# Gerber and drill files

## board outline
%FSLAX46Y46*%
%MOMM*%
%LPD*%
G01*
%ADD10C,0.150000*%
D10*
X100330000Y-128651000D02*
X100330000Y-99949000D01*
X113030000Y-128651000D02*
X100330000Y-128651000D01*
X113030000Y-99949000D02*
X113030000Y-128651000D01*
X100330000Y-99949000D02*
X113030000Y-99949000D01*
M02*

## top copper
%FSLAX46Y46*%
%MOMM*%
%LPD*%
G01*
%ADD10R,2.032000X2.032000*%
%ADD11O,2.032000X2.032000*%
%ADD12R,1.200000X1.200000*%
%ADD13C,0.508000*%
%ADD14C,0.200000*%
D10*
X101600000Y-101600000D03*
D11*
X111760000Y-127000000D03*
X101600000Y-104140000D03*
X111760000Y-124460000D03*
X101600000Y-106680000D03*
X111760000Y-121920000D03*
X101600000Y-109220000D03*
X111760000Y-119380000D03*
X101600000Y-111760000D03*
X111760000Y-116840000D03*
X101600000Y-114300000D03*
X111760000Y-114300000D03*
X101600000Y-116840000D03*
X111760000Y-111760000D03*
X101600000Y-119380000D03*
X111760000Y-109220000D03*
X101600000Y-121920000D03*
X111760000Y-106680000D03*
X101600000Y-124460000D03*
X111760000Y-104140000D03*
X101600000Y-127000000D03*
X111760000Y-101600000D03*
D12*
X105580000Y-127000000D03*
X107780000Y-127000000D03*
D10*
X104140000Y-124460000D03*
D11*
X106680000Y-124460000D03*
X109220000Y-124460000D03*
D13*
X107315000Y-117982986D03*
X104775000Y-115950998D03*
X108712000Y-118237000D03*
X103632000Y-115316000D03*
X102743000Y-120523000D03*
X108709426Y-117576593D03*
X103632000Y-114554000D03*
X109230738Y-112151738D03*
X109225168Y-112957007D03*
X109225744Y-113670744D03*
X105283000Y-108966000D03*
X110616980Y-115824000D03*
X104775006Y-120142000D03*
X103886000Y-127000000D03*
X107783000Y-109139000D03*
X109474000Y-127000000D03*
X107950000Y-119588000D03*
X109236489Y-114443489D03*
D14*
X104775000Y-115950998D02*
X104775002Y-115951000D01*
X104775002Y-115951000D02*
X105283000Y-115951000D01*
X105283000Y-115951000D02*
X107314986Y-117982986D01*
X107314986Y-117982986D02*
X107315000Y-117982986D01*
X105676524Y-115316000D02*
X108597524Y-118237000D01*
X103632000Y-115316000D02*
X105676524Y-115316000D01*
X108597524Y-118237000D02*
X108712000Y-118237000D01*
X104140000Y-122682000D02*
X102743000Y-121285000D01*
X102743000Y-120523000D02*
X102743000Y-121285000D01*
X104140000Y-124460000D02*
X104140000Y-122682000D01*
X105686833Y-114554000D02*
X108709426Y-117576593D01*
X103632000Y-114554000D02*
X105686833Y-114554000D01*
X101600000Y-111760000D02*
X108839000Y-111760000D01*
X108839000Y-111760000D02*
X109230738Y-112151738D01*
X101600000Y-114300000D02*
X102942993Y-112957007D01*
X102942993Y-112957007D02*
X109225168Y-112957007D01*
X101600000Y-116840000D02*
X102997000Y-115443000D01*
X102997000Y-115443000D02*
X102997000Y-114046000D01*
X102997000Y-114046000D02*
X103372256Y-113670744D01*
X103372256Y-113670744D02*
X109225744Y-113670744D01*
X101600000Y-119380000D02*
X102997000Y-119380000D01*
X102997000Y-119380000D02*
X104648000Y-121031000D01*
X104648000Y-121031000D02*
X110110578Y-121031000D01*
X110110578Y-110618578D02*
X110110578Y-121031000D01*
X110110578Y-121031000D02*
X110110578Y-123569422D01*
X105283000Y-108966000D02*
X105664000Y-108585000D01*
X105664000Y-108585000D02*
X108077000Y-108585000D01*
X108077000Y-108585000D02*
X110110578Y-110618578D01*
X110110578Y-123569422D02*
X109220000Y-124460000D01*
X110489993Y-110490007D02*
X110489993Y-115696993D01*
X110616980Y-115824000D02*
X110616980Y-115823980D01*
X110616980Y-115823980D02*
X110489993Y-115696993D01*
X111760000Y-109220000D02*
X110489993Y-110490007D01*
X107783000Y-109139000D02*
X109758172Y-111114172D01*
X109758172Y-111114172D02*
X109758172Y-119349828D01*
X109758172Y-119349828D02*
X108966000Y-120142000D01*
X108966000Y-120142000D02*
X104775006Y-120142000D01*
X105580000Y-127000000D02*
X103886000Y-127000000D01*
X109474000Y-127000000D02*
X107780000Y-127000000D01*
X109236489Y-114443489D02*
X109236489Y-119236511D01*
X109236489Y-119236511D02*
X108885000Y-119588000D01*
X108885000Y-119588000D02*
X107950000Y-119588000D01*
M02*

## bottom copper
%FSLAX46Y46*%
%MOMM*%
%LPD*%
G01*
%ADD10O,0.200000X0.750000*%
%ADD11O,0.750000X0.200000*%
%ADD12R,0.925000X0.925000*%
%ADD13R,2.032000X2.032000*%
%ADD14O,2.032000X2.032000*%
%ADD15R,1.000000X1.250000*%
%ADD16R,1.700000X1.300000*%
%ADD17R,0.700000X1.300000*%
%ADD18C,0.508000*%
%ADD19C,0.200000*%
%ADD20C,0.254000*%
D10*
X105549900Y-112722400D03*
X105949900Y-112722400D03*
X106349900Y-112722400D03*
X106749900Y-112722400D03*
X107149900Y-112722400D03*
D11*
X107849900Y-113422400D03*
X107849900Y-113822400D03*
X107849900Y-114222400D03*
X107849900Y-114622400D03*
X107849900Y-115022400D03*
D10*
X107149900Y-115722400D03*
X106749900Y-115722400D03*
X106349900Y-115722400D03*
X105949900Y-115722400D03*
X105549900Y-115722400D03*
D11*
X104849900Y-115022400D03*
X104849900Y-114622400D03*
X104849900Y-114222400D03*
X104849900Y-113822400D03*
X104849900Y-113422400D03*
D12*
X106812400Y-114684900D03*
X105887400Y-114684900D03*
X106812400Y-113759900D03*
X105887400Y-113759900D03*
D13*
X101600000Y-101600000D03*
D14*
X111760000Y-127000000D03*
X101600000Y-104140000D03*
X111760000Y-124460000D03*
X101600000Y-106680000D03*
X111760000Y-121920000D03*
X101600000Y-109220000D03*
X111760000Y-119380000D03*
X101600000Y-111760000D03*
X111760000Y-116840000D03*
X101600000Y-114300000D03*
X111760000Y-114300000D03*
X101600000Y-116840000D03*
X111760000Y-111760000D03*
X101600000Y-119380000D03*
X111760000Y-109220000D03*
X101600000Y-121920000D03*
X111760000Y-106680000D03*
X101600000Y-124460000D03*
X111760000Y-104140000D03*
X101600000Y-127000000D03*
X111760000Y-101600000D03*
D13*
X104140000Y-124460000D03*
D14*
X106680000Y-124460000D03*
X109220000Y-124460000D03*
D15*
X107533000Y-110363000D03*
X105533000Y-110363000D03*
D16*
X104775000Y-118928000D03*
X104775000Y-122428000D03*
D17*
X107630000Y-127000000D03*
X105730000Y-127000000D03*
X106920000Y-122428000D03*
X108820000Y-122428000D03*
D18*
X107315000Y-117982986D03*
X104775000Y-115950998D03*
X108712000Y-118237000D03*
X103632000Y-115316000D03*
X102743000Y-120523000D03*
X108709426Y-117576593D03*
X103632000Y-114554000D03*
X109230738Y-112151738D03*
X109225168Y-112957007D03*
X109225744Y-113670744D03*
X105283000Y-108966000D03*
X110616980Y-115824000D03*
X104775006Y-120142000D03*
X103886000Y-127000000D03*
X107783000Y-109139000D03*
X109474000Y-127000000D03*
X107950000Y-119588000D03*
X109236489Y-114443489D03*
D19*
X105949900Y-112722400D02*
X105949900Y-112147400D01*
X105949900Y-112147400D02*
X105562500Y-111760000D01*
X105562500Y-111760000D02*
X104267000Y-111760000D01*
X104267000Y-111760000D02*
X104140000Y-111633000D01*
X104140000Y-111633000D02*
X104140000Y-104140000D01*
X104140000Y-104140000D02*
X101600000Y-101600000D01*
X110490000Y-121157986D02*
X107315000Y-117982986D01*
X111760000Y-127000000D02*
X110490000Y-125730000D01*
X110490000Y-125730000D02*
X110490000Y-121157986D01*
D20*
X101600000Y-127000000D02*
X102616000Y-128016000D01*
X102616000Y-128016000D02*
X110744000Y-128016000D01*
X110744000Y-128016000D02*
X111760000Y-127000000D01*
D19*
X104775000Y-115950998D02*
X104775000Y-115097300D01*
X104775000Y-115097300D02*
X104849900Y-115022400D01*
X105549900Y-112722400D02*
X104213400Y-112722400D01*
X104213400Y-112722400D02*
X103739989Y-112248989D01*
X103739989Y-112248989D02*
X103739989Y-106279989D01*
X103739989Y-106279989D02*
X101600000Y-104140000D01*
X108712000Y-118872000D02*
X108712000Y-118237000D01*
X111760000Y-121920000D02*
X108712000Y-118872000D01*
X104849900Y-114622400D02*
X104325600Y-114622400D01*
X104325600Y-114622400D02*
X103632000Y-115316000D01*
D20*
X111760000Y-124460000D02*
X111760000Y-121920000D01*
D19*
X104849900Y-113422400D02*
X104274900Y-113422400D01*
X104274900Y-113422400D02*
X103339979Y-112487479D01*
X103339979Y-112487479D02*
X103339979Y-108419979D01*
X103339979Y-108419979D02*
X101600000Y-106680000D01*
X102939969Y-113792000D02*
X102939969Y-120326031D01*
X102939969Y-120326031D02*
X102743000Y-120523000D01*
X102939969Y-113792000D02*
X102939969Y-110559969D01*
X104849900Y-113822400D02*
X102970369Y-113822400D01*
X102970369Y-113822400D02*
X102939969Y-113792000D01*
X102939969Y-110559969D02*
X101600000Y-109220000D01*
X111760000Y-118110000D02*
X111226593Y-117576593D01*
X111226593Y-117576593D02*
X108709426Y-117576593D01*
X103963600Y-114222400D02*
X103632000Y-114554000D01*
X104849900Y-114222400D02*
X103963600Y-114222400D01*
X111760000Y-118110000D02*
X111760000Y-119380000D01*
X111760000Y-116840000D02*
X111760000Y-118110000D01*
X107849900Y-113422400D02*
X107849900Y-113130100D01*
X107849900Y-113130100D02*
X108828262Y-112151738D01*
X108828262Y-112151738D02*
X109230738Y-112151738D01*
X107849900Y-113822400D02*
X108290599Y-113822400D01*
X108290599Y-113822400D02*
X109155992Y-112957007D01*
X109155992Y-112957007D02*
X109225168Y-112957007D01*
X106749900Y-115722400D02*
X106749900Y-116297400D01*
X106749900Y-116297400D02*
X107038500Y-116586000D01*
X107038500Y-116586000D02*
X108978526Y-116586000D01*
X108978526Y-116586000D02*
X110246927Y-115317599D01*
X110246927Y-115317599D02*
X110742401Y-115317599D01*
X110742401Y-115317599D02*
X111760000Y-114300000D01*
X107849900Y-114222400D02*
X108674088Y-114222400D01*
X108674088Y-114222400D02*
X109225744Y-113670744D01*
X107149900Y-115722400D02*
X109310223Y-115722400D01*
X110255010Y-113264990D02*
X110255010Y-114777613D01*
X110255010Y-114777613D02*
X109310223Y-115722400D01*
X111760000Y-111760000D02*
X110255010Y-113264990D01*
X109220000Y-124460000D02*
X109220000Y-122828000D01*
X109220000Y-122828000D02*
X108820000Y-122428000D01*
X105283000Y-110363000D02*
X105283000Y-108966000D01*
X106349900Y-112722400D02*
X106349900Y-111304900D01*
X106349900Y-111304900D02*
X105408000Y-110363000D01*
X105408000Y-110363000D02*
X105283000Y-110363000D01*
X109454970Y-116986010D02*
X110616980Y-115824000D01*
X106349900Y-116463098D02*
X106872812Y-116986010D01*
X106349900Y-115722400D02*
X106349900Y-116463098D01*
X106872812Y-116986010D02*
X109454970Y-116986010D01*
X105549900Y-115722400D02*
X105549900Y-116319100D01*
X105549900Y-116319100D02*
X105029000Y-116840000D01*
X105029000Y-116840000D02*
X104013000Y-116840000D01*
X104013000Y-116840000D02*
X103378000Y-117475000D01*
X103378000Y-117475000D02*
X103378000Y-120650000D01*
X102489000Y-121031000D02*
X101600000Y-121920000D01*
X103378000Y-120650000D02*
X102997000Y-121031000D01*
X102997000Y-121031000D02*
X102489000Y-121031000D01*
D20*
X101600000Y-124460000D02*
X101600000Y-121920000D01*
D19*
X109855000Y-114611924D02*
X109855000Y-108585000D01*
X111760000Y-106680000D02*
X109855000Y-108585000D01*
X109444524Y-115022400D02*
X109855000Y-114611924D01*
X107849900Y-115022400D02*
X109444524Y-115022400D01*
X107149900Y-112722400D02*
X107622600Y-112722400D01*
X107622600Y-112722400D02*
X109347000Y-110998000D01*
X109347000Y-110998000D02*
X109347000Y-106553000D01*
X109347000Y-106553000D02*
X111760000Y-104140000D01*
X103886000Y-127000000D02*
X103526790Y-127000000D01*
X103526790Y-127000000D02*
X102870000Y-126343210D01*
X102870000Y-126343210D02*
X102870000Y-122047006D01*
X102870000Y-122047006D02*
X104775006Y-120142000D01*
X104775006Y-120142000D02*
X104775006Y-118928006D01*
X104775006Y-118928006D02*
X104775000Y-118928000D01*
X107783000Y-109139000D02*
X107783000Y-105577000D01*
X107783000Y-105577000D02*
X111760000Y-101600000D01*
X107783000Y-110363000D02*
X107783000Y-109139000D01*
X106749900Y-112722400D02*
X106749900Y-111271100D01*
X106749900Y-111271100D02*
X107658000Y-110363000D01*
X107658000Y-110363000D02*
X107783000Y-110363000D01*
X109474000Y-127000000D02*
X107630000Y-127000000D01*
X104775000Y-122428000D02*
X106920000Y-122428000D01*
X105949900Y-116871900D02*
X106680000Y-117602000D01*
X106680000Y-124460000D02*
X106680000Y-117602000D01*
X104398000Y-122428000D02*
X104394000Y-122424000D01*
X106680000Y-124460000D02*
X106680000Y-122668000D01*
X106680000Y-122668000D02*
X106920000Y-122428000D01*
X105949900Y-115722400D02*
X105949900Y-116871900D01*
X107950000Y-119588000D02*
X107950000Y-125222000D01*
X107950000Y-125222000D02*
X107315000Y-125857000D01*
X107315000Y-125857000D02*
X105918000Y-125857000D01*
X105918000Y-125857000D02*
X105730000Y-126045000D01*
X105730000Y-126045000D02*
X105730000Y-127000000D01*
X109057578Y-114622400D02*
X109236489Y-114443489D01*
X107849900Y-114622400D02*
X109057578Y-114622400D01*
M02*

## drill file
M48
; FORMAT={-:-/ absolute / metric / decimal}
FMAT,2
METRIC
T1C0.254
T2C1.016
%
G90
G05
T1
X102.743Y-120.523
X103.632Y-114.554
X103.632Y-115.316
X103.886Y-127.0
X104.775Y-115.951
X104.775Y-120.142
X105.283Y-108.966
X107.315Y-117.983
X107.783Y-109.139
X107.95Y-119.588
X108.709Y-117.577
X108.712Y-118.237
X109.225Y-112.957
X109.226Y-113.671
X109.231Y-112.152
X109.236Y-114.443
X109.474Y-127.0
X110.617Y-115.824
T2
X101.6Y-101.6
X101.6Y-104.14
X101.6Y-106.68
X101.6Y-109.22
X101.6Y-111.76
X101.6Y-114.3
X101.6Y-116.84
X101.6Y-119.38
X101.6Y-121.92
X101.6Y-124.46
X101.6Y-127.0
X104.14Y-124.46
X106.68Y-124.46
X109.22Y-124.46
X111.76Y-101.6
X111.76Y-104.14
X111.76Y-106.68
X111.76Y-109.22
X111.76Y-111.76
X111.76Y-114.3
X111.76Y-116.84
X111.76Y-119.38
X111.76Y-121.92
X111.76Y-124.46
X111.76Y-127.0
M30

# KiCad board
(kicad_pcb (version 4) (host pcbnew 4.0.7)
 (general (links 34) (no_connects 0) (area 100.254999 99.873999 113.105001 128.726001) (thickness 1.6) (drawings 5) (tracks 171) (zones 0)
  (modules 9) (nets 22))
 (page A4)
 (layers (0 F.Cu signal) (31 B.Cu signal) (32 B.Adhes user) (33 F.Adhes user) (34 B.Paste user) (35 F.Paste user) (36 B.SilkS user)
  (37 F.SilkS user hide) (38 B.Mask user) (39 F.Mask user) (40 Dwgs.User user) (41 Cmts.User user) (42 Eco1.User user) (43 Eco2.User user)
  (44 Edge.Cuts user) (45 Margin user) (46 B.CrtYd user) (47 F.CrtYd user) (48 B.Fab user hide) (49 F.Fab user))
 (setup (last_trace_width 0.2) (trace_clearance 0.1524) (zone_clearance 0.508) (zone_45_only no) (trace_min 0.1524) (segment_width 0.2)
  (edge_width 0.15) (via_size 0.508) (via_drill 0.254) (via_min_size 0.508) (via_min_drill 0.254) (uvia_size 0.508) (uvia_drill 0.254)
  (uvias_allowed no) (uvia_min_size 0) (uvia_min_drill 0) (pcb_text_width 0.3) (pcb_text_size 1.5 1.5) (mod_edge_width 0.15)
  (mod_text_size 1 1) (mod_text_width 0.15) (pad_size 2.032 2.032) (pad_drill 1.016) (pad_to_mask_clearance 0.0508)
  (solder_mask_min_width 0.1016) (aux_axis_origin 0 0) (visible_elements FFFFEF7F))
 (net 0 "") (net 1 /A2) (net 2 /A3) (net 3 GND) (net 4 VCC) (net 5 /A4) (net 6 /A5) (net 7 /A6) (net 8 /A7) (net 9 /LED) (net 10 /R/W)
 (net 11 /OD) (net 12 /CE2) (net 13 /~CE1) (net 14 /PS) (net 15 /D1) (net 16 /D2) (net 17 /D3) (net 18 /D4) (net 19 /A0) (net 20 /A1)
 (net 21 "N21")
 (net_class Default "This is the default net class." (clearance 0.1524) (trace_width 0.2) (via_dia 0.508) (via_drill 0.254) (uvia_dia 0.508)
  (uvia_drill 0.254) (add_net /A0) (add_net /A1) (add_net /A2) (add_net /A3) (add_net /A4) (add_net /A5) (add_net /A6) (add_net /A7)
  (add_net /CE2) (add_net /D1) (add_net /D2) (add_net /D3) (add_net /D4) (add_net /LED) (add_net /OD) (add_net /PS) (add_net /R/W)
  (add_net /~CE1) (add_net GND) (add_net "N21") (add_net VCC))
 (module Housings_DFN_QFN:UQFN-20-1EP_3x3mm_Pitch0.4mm (layer B.Cu) (at 106.3499 114.2224 270) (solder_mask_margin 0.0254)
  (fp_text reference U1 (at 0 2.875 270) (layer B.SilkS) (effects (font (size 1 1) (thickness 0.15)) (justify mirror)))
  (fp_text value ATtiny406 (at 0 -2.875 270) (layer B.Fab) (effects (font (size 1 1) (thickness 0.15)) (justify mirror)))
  (pad 1 smd oval (at -1.5 0.8 270) (size 0.75 0.2) (layers B.Cu B.Paste B.Mask) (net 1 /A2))
  (pad 2 smd oval (at -1.5 0.4 270) (size 0.75 0.2) (layers B.Cu B.Paste B.Mask) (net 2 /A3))
  (pad 3 smd oval (at -1.5 0 270) (size 0.75 0.2) (layers B.Cu B.Paste B.Mask) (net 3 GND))
  (pad 4 smd oval (at -1.5 -0.4 270) (size 0.75 0.2) (layers B.Cu B.Paste B.Mask) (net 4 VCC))
  (pad 5 smd oval (at -1.5 -0.8 270) (size 0.75 0.2) (layers B.Cu B.Paste B.Mask) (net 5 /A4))
  (pad 6 smd oval (at -0.8 -1.5 180) (size 0.75 0.2) (layers B.Cu B.Paste B.Mask) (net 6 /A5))
  (pad 7 smd oval (at -0.4 -1.5 180) (size 0.75 0.2) (layers B.Cu B.Paste B.Mask) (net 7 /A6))
  (pad 8 smd oval (at 0 -1.5 180) (size 0.75 0.2) (layers B.Cu B.Paste B.Mask) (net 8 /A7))
  (pad 9 smd oval (at 0.4 -1.5 180) (size 0.75 0.2) (layers B.Cu B.Paste B.Mask) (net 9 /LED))
  (pad 10 smd oval (at 0.8 -1.5 180) (size 0.75 0.2) (layers B.Cu B.Paste B.Mask) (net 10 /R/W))
  (pad 11 smd oval (at 1.5 -0.8 270) (size 0.75 0.2) (layers B.Cu B.Paste B.Mask) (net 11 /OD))
  (pad 12 smd oval (at 1.5 -0.4 270) (size 0.75 0.2) (layers B.Cu B.Paste B.Mask) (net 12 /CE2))
  (pad 13 smd oval (at 1.5 0 270) (size 0.75 0.2) (layers B.Cu B.Paste B.Mask) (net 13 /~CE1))
  (pad 14 smd oval (at 1.5 0.4 270) (size 0.75 0.2) (layers B.Cu B.Paste B.Mask) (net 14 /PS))
  (pad 15 smd oval (at 1.5 0.8 270) (size 0.75 0.2) (layers B.Cu B.Paste B.Mask) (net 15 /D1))
  (pad 16 smd oval (at 0.8 1.5 180) (size 0.75 0.2) (layers B.Cu B.Paste B.Mask) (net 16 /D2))
  (pad 17 smd oval (at 0.4 1.5 180) (size 0.75 0.2) (layers B.Cu B.Paste B.Mask) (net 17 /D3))
  (pad 18 smd oval (at 0 1.5 180) (size 0.75 0.2) (layers B.Cu B.Paste B.Mask) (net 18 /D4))
  (pad 19 smd oval (at -0.4 1.5 180) (size 0.75 0.2) (layers B.Cu B.Paste B.Mask) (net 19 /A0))
  (pad 20 smd oval (at -0.8 1.5 180) (size 0.75 0.2) (layers B.Cu B.Paste B.Mask) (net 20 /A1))
  (pad 21 smd rect (at 0.4625 -0.4625 270) (size 0.925 0.925) (layers B.Cu B.Paste B.Mask) (solder_paste_margin_ratio -0.2))
  (pad 21 smd rect (at 0.4625 0.4625 270) (size 0.925 0.925) (layers B.Cu B.Paste B.Mask) (solder_paste_margin_ratio -0.2))
  (pad 21 smd rect (at -0.4625 -0.4625 270) (size 0.925 0.925) (layers B.Cu B.Paste B.Mask) (solder_paste_margin_ratio -0.2))
  (pad 21 smd rect (at -0.4625 0.4625 270) (size 0.925 0.925) (layers B.Cu B.Paste B.Mask) (solder_paste_margin_ratio -0.2)))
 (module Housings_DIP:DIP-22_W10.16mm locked (layer F.Cu) (at 101.6 101.6)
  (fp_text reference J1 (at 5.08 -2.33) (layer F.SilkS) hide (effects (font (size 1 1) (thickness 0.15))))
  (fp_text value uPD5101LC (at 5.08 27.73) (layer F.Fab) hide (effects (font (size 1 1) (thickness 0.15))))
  (pad 1 thru_hole rect (at 0 0) (size 2.032 2.032) (drill 1.016) (layers *.Cu *.Mask) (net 2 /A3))
  (pad 12 thru_hole oval (at 10.16 25.4) (size 2.032 2.032) (drill 1.016) (layers *.Cu *.Mask) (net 16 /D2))
  (pad 2 thru_hole oval (at 0 2.54) (size 2.032 2.032) (drill 1.016) (layers *.Cu *.Mask) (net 1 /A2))
  (pad 13 thru_hole oval (at 10.16 22.86) (size 2.032 2.032) (drill 1.016) (layers *.Cu *.Mask) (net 17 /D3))
  (pad 3 thru_hole oval (at 0 5.08) (size 2.032 2.032) (drill 1.016) (layers *.Cu *.Mask) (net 20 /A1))
  (pad 14 thru_hole oval (at 10.16 20.32) (size 2.032 2.032) (drill 1.016) (layers *.Cu *.Mask) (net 17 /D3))
  (pad 4 thru_hole oval (at 0 7.62) (size 2.032 2.032) (drill 1.016) (layers *.Cu *.Mask) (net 19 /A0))
  (pad 15 thru_hole oval (at 10.16 17.78) (size 2.032 2.032) (drill 1.016) (layers *.Cu *.Mask) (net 18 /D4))
  (pad 5 thru_hole oval (at 0 10.16) (size 2.032 2.032) (drill 1.016) (layers *.Cu *.Mask) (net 6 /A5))
  (pad 16 thru_hole oval (at 10.16 15.24) (size 2.032 2.032) (drill 1.016) (layers *.Cu *.Mask) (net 18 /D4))
  (pad 6 thru_hole oval (at 0 12.7) (size 2.032 2.032) (drill 1.016) (layers *.Cu *.Mask) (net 7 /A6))
  (pad 17 thru_hole oval (at 10.16 12.7) (size 2.032 2.032) (drill 1.016) (layers *.Cu *.Mask) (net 12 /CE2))
  (pad 7 thru_hole oval (at 0 15.24) (size 2.032 2.032) (drill 1.016) (layers *.Cu *.Mask) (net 8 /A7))
  (pad 18 thru_hole oval (at 10.16 10.16) (size 2.032 2.032) (drill 1.016) (layers *.Cu *.Mask) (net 11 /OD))
  (pad 8 thru_hole oval (at 0 17.78) (size 2.032 2.032) (drill 1.016) (layers *.Cu *.Mask) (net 3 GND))
  (pad 19 thru_hole oval (at 10.16 7.62) (size 2.032 2.032) (drill 1.016) (layers *.Cu *.Mask) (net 13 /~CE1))
  (pad 9 thru_hole oval (at 0 20.32) (size 2.032 2.032) (drill 1.016) (layers *.Cu *.Mask) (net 15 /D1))
  (pad 20 thru_hole oval (at 10.16 5.08) (size 2.032 2.032) (drill 1.016) (layers *.Cu *.Mask) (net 10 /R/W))
  (pad 10 thru_hole oval (at 0 22.86) (size 2.032 2.032) (drill 1.016) (layers *.Cu *.Mask) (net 15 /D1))
  (pad 21 thru_hole oval (at 10.16 2.54) (size 2.032 2.032) (drill 1.016) (layers *.Cu *.Mask) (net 5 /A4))
  (pad 11 thru_hole oval (at 0 25.4) (size 2.032 2.032) (drill 1.016) (layers *.Cu *.Mask) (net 16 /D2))
  (pad 22 thru_hole oval (at 10.16 0) (size 2.032 2.032) (drill 1.016) (layers *.Cu *.Mask) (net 4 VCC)))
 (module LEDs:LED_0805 (layer F.Cu) (at 106.68 127 180)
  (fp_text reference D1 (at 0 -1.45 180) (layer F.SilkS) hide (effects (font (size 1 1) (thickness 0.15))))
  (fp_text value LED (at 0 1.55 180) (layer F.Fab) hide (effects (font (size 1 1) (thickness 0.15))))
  (pad 2 smd rect (at 1.1 0) (size 1.2 1.2) (layers F.Cu F.Paste F.Mask) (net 4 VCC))
  (pad 1 smd rect (at -1.1 0) (size 1.2 1.2) (layers F.Cu F.Paste F.Mask) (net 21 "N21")))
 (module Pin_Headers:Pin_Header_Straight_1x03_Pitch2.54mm (layer F.Cu) (at 104.14 124.46 90)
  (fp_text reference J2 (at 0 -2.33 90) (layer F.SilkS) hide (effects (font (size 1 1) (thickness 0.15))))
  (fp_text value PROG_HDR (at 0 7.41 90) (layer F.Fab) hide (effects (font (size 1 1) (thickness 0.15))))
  (pad 1 thru_hole rect (at 0 0 90) (size 2.032 2.032) (drill 1.016) (layers *.Cu *.Mask) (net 19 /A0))
  (pad 2 thru_hole oval (at 0 2.54 90) (size 2.032 2.032) (drill 1.016) (layers *.Cu *.Mask) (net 14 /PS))
  (pad 3 thru_hole oval (at 0 5.08 90) (size 2.032 2.032) (drill 1.016) (layers *.Cu *.Mask) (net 3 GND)))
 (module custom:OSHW (layer F.Cu) (at 106.553 120.269 270)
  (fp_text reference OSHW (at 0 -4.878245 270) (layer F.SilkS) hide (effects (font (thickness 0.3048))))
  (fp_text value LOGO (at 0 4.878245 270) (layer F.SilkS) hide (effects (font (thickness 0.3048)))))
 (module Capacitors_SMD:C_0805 (layer B.Cu) (at 106.533 110.363 180)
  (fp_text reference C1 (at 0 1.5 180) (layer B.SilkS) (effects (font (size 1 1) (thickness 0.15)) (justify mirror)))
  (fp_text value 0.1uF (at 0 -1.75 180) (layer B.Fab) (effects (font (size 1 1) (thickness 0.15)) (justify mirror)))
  (pad 1 smd rect (at -1 0 180) (size 1 1.25) (layers B.Cu B.Paste B.Mask) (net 4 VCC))
  (pad 2 smd rect (at 1 0 180) (size 1 1.25) (layers B.Cu B.Paste B.Mask) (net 3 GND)))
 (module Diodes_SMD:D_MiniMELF (layer B.Cu) (at 104.775 120.678 270)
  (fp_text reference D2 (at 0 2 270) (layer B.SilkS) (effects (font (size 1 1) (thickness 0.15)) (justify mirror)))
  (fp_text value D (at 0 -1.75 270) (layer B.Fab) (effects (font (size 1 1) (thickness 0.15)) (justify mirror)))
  (pad 1 smd rect (at -1.75 0 270) (size 1.3 1.7) (layers B.Cu B.Paste B.Mask) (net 4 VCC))
  (pad 2 smd rect (at 1.75 0 270) (size 1.3 1.7) (layers B.Cu B.Paste B.Mask) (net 14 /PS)))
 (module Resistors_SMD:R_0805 (layer B.Cu) (at 106.68 127 180)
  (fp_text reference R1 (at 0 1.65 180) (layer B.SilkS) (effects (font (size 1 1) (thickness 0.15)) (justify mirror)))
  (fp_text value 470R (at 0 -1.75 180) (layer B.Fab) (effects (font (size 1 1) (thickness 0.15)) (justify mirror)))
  (pad 1 smd rect (at -0.95 0 180) (size 0.7 1.3) (layers B.Cu B.Paste B.Mask) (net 21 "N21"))
  (pad 2 smd rect (at 0.95 0 180) (size 0.7 1.3) (layers B.Cu B.Paste B.Mask) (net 9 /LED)))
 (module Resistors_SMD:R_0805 (layer B.Cu) (at 107.87 122.428)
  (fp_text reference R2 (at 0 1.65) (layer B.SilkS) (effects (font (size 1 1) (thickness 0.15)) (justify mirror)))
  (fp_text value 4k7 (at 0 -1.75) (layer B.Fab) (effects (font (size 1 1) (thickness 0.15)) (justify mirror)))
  (pad 1 smd rect (at -0.95 0) (size 0.7 1.3) (layers B.Cu B.Paste B.Mask) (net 14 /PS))
  (pad 2 smd rect (at 0.95 0) (size 0.7 1.3) (layers B.Cu B.Paste B.Mask) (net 3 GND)))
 (gr_line (start 100.33 128.651) (end 100.33 99.949) (layer Edge.Cuts) (width 0.15))
 (gr_line (start 113.03 128.651) (end 100.33 128.651) (layer Edge.Cuts) (width 0.15))
 (gr_line (start 113.03 99.949) (end 113.03 128.651) (layer Edge.Cuts) (width 0.15))
 (gr_line (start 100.33 99.949) (end 113.03 99.949) (layer Edge.Cuts) (width 0.15))
 (segment (start 105.9499 112.7224) (end 105.9499 112.1474) (width 0.2) (layer B.Cu) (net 2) (status 10))
 (segment (start 105.9499 112.1474) (end 105.5625 111.76) (width 0.2) (layer B.Cu) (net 2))
 (segment (start 105.5625 111.76) (end 104.267 111.76) (width 0.2) (layer B.Cu) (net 2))
 (segment (start 104.267 111.76) (end 104.14 111.633) (width 0.2) (layer B.Cu) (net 2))
 (segment (start 104.14 111.633) (end 104.14 104.14) (width 0.2) (layer B.Cu) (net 2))
 (segment (start 104.14 104.14) (end 101.6 101.6) (width 0.2) (layer B.Cu) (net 2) (status 20))
 (segment (start 104.775 115.950998) (end 104.775002 115.951) (width 0.2) (layer F.Cu) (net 16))
 (segment (start 104.775002 115.951) (end 105.283 115.951) (width 0.2) (layer F.Cu) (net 16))
 (segment (start 105.283 115.951) (end 107.314986 117.982986) (width 0.2) (layer F.Cu) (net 16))
 (segment (start 107.314986 117.982986) (end 107.315 117.982986) (width 0.2) (layer F.Cu) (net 16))
 (segment (start 110.49 121.157986) (end 107.315 117.982986) (width 0.2) (layer B.Cu) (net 16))
 (segment (start 111.76 127) (end 110.49 125.73) (width 0.2) (layer B.Cu) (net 16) (status 10))
 (segment (start 110.49 125.73) (end 110.49 121.157986) (width 0.2) (layer B.Cu) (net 16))
 (via (at 107.315 117.982986) (size 0.508) (drill 0.254) (layers F.Cu B.Cu) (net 16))
 (segment (start 101.6 127) (end 102.616 128.016) (width 0.254) (layer B.Cu) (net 16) (status 10))
 (segment (start 102.616 128.016) (end 110.744 128.016) (width 0.254) (layer B.Cu) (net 16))
 (segment (start 110.744 128.016) (end 111.76 127) (width 0.254) (layer B.Cu) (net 16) (status 20))
 (segment (start 104.775 115.950998) (end 104.775 115.0973) (width 0.2) (layer B.Cu) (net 16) (status 20))
 (segment (start 104.775 115.0973) (end 104.8499 115.0224) (width 0.2) (layer B.Cu) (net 16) (status 30))
 (via (at 104.775 115.950998) (size 0.508) (drill 0.254) (layers F.Cu B.Cu) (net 16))
 (segment (start 105.5499 112.7224) (end 104.2134 112.7224) (width 0.2) (layer B.Cu) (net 1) (status 10))
 (segment (start 104.2134 112.7224) (end 103.739989 112.248989) (width 0.2) (layer B.Cu) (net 1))
 (segment (start 103.739989 112.248989) (end 103.739989 106.279989) (width 0.2) (layer B.Cu) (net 1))
 (segment (start 103.739989 106.279989) (end 101.6 104.14) (width 0.2) (layer B.Cu) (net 1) (status 20))
 (segment (start 105.676524 115.316) (end 108.597524 118.237) (width 0.2) (layer F.Cu) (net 17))
 (segment (start 103.632 115.316) (end 105.676524 115.316) (width 0.2) (layer F.Cu) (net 17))
 (segment (start 108.712 118.872) (end 108.712 118.237) (width 0.2) (layer B.Cu) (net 17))
 (via (at 108.712 118.237) (size 0.508) (drill 0.254) (layers F.Cu B.Cu) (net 17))
 (segment (start 108.597524 118.237) (end 108.712 118.237) (width 0.2) (layer F.Cu) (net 17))
 (segment (start 111.76 121.92) (end 108.712 118.872) (width 0.2) (layer B.Cu) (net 17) (status 10))
 (segment (start 104.8499 114.6224) (end 104.3256 114.6224) (width 0.2) (layer B.Cu) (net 17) (status 10))
 (segment (start 104.3256 114.6224) (end 103.632 115.316) (width 0.2) (layer B.Cu) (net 17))
 (via (at 103.632 115.316) (size 0.508) (drill 0.254) (layers F.Cu B.Cu) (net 17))
 (segment (start 111.76 124.46) (end 111.76 121.92) (width 0.254) (layer B.Cu) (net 17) (status 30))
 (segment (start 104.8499 113.4224) (end 104.2749 113.4224) (width 0.2) (layer B.Cu) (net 20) (status 10))
 (segment (start 104.2749 113.4224) (end 103.339979 112.487479) (width 0.2) (layer B.Cu) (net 20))
 (segment (start 103.339979 112.487479) (end 103.339979 108.419979) (width 0.2) (layer B.Cu) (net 20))
 (segment (start 103.339979 108.419979) (end 101.6 106.68) (width 0.2) (layer B.Cu) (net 20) (status 20))
 (segment (start 104.14 122.682) (end 102.743 121.285) (width 0.2) (layer F.Cu) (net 19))
 (segment (start 102.743 120.523) (end 102.743 121.285) (width 0.2) (layer F.Cu) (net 19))
 (segment (start 102.939969 113.792) (end 102.939969 120.326031) (width 0.2) (layer B.Cu) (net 19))
 (segment (start 102.939969 120.326031) (end 102.743 120.523) (width 0.2) (layer B.Cu) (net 19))
 (via (at 102.743 120.523) (size 0.508) (drill 0.254) (layers F.Cu B.Cu) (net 19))
 (segment (start 102.939969 113.792) (end 102.939969 110.559969) (width 0.2) (layer B.Cu) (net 19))
 (segment (start 104.8499 113.8224) (end 102.970369 113.8224) (width 0.2) (layer B.Cu) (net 19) (status 10))
 (segment (start 102.970369 113.8224) (end 102.939969 113.792) (width 0.2) (layer B.Cu) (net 19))
 (segment (start 104.14 124.46) (end 104.14 122.682) (width 0.2) (layer F.Cu) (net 19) (status 10))
 (segment (start 102.939969 110.559969) (end 101.6 109.22) (width 0.2) (layer B.Cu) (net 19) (status 20))
 (via (at 108.709426 117.576593) (size 0.508) (drill 0.254) (layers F.Cu B.Cu) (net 18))
 (segment (start 111.76 118.11) (end 111.226593 117.576593) (width 0.2) (layer B.Cu) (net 18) (status 20))
 (segment (start 105.686833 114.554) (end 108.709426 117.576593) (width 0.2) (layer F.Cu) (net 18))
 (segment (start 111.226593 117.576593) (end 108.709426 117.576593) (width 0.2) (layer B.Cu) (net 18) (status 10))
 (segment (start 103.632 114.554) (end 105.686833 114.554) (width 0.2) (layer F.Cu) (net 18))
 (segment (start 103.9636 114.2224) (end 103.632 114.554) (width 0.2) (layer B.Cu) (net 18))
 (segment (start 104.8499 114.2224) (end 103.9636 114.2224) (width 0.2) (layer B.Cu) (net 18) (status 10))
 (via (at 103.632 114.554) (size 0.508) (drill 0.254) (layers F.Cu B.Cu) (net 18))
 (segment (start 111.76 118.11) (end 111.76 119.38) (width 0.2) (layer B.Cu) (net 18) (status 20))
 (segment (start 111.76 116.84) (end 111.76 118.11) (width 0.2) (layer B.Cu) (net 18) (status 10))
 (segment (start 101.6 111.76) (end 108.839 111.76) (width 0.2) (layer F.Cu) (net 6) (status 10))
 (segment (start 108.839 111.76) (end 109.230738 112.151738) (width 0.2) (layer F.Cu) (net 6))
 (segment (start 107.8499 113.4224) (end 107.8499 113.1301) (width 0.2) (layer B.Cu) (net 6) (status 10))
 (segment (start 107.8499 113.1301) (end 108.828262 112.151738) (width 0.2) (layer B.Cu) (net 6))
 (segment (start 108.828262 112.151738) (end 109.230738 112.151738) (width 0.2) (layer B.Cu) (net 6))
 (via (at 109.230738 112.151738) (size 0.508) (drill 0.254) (layers F.Cu B.Cu) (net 6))
 (segment (start 101.6 114.3) (end 102.942993 112.957007) (width 0.2) (layer F.Cu) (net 7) (status 10))
 (segment (start 102.942993 112.957007) (end 109.225168 112.957007) (width 0.2) (layer F.Cu) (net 7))
 (segment (start 107.8499 113.8224) (end 108.290599 113.8224) (width 0.2) (layer B.Cu) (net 7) (status 10))
 (segment (start 108.290599 113.8224) (end 109.155992 112.957007) (width 0.2) (layer B.Cu) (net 7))
 (segment (start 109.155992 112.957007) (end 109.225168 112.957007) (width 0.2) (layer B.Cu) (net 7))
 (via (at 109.225168 112.957007) (size 0.508) (drill 0.254) (layers F.Cu B.Cu) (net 7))
 (segment (start 106.7499 115.7224) (end 106.7499 116.2974) (width 0.2) (layer B.Cu) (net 12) (status 10))
 (segment (start 106.7499 116.2974) (end 107.0385 116.586) (width 0.2) (layer B.Cu) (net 12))
 (segment (start 107.0385 116.586) (end 108.978526 116.586) (width 0.2) (layer B.Cu) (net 12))
 (segment (start 108.978526 116.586) (end 110.246927 115.317599) (width 0.2) (layer B.Cu) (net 12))
 (segment (start 110.246927 115.317599) (end 110.742401 115.317599) (width 0.2) (layer B.Cu) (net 12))
 (segment (start 110.742401 115.317599) (end 111.76 114.3) (width 0.2) (layer B.Cu) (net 12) (status 20))
 (segment (start 101.6 116.84) (end 102.997 115.443) (width 0.2) (layer F.Cu) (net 8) (status 10))
 (segment (start 102.997 115.443) (end 102.997 114.046) (width 0.2) (layer F.Cu) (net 8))
 (segment (start 102.997 114.046) (end 103.372256 113.670744) (width 0.2) (layer F.Cu) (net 8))
 (segment (start 103.372256 113.670744) (end 109.225744 113.670744) (width 0.2) (layer F.Cu) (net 8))
 (segment (start 107.8499 114.2224) (end 108.674088 114.2224) (width 0.2) (layer B.Cu) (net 8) (status 10))
 (segment (start 108.674088 114.2224) (end 109.225744 113.670744) (width 0.2) (layer B.Cu) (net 8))
 (via (at 109.225744 113.670744) (size 0.508) (drill 0.254) (layers F.Cu B.Cu) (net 8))
 (segment (start 107.1499 115.7224) (end 109.310223 115.7224) (width 0.2) (layer B.Cu) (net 11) (status 10))
 (segment (start 110.25501 113.26499) (end 110.25501 114.777613) (width 0.2) (layer B.Cu) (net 11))
 (segment (start 110.25501 114.777613) (end 109.310223 115.7224) (width 0.2) (layer B.Cu) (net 11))
 (segment (start 111.76 111.76) (end 110.25501 113.26499) (width 0.2) (layer B.Cu) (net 11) (status 10))
 (segment (start 101.6 119.38) (end 102.997 119.38) (width 0.2) (layer F.Cu) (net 3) (status 10))
 (segment (start 102.997 119.38) (end 104.648 121.031) (width 0.2) (layer F.Cu) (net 3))
 (segment (start 104.648 121.031) (end 110.110578 121.031) (width 0.2) (layer F.Cu) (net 3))
 (segment (start 110.110578 110.618578) (end 110.110578 121.031) (width 0.2) (layer F.Cu) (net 3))
 (segment (start 110.110578 121.031) (end 110.110578 123.569422) (width 0.2) (layer F.Cu) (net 3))
 (segment (start 105.283 108.966) (end 105.664 108.585) (width 0.2) (layer F.Cu) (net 3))
 (segment (start 105.664 108.585) (end 108.077 108.585) (width 0.2) (layer F.Cu) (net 3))
 (segment (start 108.077 108.585) (end 110.110578 110.618578) (width 0.2) (layer F.Cu) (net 3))
 (segment (start 110.110578 123.569422) (end 109.22 124.46) (width 0.2) (layer F.Cu) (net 3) (status 20))
 (segment (start 109.22 124.46) (end 109.22 122.828) (width 0.2) (layer B.Cu) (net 3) (status 10))
 (segment (start 109.22 122.828) (end 108.82 122.428) (width 0.2) (layer B.Cu) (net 3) (status 20))
 (via (at 105.283 108.966) (size 0.508) (drill 0.254) (layers F.Cu B.Cu) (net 3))
 (segment (start 105.283 110.363) (end 105.283 108.966) (width 0.2) (layer B.Cu) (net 3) (status 10))
 (segment (start 106.3499 112.7224) (end 106.3499 111.3049) (width 0.2) (layer B.Cu) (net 3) (status 10))
 (segment (start 106.3499 111.3049) (end 105.408 110.363) (width 0.2) (layer B.Cu) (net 3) (status 20))
 (segment (start 105.408 110.363) (end 105.283 110.363) (width 0.2) (layer B.Cu) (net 3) (status 30))
 (segment (start 110.489993 110.490007) (end 110.489993 115.696993) (width 0.2) (layer F.Cu) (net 13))
 (segment (start 110.61698 115.824) (end 110.61698 115.82398) (width 0.2) (layer F.Cu) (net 13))
 (segment (start 110.61698 115.82398) (end 110.489993 115.696993) (width 0.2) (layer F.Cu) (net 13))
 (segment (start 111.76 109.22) (end 110.489993 110.490007) (width 0.2) (layer F.Cu) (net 13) (status 10))
 (segment (start 109.45497 116.98601) (end 110.61698 115.824) (width 0.2) (layer B.Cu) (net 13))
 (segment (start 106.3499 116.463098) (end 106.872812 116.98601) (width 0.2) (layer B.Cu) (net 13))
 (segment (start 106.3499 115.7224) (end 106.3499 116.463098) (width 0.2) (layer B.Cu) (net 13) (status 10))
 (via (at 110.61698 115.824) (size 0.508) (drill 0.254) (layers F.Cu B.Cu) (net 13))
 (segment (start 106.872812 116.98601) (end 109.45497 116.98601) (width 0.2) (layer B.Cu) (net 13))
 (segment (start 105.5499 115.7224) (end 105.5499 116.3191) (width 0.2) (layer B.Cu) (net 15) (status 10))
 (segment (start 105.5499 116.3191) (end 105.029 116.84) (width 0.2) (layer B.Cu) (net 15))
 (segment (start 105.029 116.84) (end 104.013 116.84) (width 0.2) (layer B.Cu) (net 15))
 (segment (start 104.013 116.84) (end 103.378 117.475) (width 0.2) (layer B.Cu) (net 15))
 (segment (start 103.378 117.475) (end 103.378 120.65) (width 0.2) (layer B.Cu) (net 15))
 (segment (start 102.489 121.031) (end 101.6 121.92) (width 0.2) (layer B.Cu) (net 15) (status 20))
 (segment (start 103.378 120.65) (end 102.997 121.031) (width 0.2) (layer B.Cu) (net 15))
 (segment (start 102.997 121.031) (end 102.489 121.031) (width 0.2) (layer B.Cu) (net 15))
 (segment (start 101.6 124.46) (end 101.6 121.92) (width 0.254) (layer B.Cu) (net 15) (status 30))
 (segment (start 109.855 114.611924) (end 109.855 108.585) (width 0.2) (layer B.Cu) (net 10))
 (segment (start 111.76 106.68) (end 109.855 108.585) (width 0.2) (layer B.Cu) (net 10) (status 10))
 (segment (start 109.444524 115.0224) (end 109.855 114.611924) (width 0.2) (layer B.Cu) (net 10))
 (segment (start 107.8499 115.0224) (end 109.444524 115.0224) (width 0.2) (layer B.Cu) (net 10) (status 10))
 (segment (start 107.1499 112.7224) (end 107.6226 112.7224) (width 0.2) (layer B.Cu) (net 5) (status 10))
 (segment (start 107.6226 112.7224) (end 109.347 110.998) (width 0.2) (layer B.Cu) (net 5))
 (segment (start 109.347 110.998) (end 109.347 106.553) (width 0.2) (layer B.Cu) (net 5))
 (segment (start 109.347 106.553) (end 111.76 104.14) (width 0.2) (layer B.Cu) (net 5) (status 20))
 (segment (start 107.783 109.139) (end 109.758172 111.114172) (width 0.2) (layer F.Cu) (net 4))
 (segment (start 109.758172 111.114172) (end 109.758172 119.349828) (width 0.2) (layer F.Cu) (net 4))
 (segment (start 109.758172 119.349828) (end 108.966 120.142) (width 0.2) (layer F.Cu) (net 4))
 (segment (start 108.966 120.142) (end 104.775006 120.142) (width 0.2) (layer F.Cu) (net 4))
 (segment (start 103.886 127) (end 103.52679 127) (width 0.2) (layer B.Cu) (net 4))
 (segment (start 103.52679 127) (end 102.87 126.34321) (width 0.2) (layer B.Cu) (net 4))
 (segment (start 102.87 126.34321) (end 102.87 122.047006) (width 0.2) (layer B.Cu) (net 4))
 (segment (start 102.87 122.047006) (end 104.775006 120.142) (width 0.2) (layer B.Cu) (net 4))
 (segment (start 104.775006 120.142) (end 104.775006 118.928006) (width 0.2) (layer B.Cu) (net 4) (status 20))
 (segment (start 104.775006 118.928006) (end 104.775 118.928) (width 0.2) (layer B.Cu) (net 4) (status 30))
 (via (at 104.775006 120.142) (size 0.508) (drill 0.254) (layers F.Cu B.Cu) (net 4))
 (segment (start 105.58 127) (end 103.886 127) (width 0.2) (layer F.Cu) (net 4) (status 10))
 (via (at 103.886 127) (size 0.508) (drill 0.254) (layers F.Cu B.Cu) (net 4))
 (segment (start 107.783 109.139) (end 107.783 105.577) (width 0.2) (layer B.Cu) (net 4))
 (segment (start 107.783 105.577) (end 111.76 101.6) (width 0.2) (layer B.Cu) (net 4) (status 20))
 (via (at 107.783 109.139) (size 0.508) (drill 0.254) (layers F.Cu B.Cu) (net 4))
 (segment (start 107.783 110.363) (end 107.783 109.139) (width 0.2) (layer B.Cu) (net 4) (status 10))
 (segment (start 106.7499 112.7224) (end 106.7499 111.2711) (width 0.2) (layer B.Cu) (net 4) (status 10))
 (segment (start 106.7499 111.2711) (end 107.658 110.363) (width 0.2) (layer B.Cu) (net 4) (status 20))
 (segment (start 107.658 110.363) (end 107.783 110.363) (width 0.2) (layer B.Cu) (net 4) (status 30))
 (segment (start 109.474 127) (end 107.78 127) (width 0.2) (layer F.Cu) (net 21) (status 20))
 (segment (start 109.474 127) (end 107.63 127) (width 0.2) (layer B.Cu) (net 21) (status 20))
 (via (at 109.474 127) (size 0.508) (drill 0.254) (layers F.Cu B.Cu) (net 21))
 (segment (start 104.775 122.428) (end 106.92 122.428) (width 0.2) (layer B.Cu) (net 14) (status 30))
 (segment (start 105.9499 116.8719) (end 106.68 117.602) (width 0.2) (layer B.Cu) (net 14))
 (segment (start 106.68 124.46) (end 106.68 117.602) (width 0.2) (layer B.Cu) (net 14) (status 10))
 (segment (start 104.398 122.428) (end 104.394 122.424) (width 0.2) (layer B.Cu) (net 14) (status 30))
 (segment (start 106.68 124.46) (end 106.68 122.668) (width 0.2) (layer B.Cu) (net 14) (status 30))
 (segment (start 106.68 122.668) (end 106.92 122.428) (width 0.2) (layer B.Cu) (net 14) (status 30))
 (segment (start 105.9499 115.7224) (end 105.9499 116.8719) (width 0.2) (layer B.Cu) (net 14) (status 10))
 (segment (start 107.95 119.588) (end 107.95 125.222) (width 0.2) (layer B.Cu) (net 9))
 (segment (start 107.95 125.222) (end 107.315 125.857) (width 0.2) (layer B.Cu) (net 9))
 (segment (start 107.315 125.857) (end 105.918 125.857) (width 0.2) (layer B.Cu) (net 9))
 (segment (start 105.918 125.857) (end 105.73 126.045) (width 0.2) (layer B.Cu) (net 9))
 (segment (start 105.73 126.045) (end 105.73 127) (width 0.2) (layer B.Cu) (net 9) (status 20))
 (segment (start 109.236489 114.443489) (end 109.236489 119.236511) (width 0.2) (layer F.Cu) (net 9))
 (segment (start 109.236489 119.236511) (end 108.885 119.588) (width 0.2) (layer F.Cu) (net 9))
 (segment (start 108.885 119.588) (end 107.95 119.588) (width 0.2) (layer F.Cu) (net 9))
 (via (at 107.95 119.588) (size 0.508) (drill 0.254) (layers F.Cu B.Cu) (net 9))
 (via (at 109.236489 114.443489) (size 0.508) (drill 0.254) (layers F.Cu B.Cu) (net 9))
 (segment (start 109.057578 114.6224) (end 109.236489 114.443489) (width 0.2) (layer B.Cu) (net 9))
 (segment (start 107.8499 114.6224) (end 109.057578 114.6224) (width 0.2) (layer B.Cu) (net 9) (status 10)))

